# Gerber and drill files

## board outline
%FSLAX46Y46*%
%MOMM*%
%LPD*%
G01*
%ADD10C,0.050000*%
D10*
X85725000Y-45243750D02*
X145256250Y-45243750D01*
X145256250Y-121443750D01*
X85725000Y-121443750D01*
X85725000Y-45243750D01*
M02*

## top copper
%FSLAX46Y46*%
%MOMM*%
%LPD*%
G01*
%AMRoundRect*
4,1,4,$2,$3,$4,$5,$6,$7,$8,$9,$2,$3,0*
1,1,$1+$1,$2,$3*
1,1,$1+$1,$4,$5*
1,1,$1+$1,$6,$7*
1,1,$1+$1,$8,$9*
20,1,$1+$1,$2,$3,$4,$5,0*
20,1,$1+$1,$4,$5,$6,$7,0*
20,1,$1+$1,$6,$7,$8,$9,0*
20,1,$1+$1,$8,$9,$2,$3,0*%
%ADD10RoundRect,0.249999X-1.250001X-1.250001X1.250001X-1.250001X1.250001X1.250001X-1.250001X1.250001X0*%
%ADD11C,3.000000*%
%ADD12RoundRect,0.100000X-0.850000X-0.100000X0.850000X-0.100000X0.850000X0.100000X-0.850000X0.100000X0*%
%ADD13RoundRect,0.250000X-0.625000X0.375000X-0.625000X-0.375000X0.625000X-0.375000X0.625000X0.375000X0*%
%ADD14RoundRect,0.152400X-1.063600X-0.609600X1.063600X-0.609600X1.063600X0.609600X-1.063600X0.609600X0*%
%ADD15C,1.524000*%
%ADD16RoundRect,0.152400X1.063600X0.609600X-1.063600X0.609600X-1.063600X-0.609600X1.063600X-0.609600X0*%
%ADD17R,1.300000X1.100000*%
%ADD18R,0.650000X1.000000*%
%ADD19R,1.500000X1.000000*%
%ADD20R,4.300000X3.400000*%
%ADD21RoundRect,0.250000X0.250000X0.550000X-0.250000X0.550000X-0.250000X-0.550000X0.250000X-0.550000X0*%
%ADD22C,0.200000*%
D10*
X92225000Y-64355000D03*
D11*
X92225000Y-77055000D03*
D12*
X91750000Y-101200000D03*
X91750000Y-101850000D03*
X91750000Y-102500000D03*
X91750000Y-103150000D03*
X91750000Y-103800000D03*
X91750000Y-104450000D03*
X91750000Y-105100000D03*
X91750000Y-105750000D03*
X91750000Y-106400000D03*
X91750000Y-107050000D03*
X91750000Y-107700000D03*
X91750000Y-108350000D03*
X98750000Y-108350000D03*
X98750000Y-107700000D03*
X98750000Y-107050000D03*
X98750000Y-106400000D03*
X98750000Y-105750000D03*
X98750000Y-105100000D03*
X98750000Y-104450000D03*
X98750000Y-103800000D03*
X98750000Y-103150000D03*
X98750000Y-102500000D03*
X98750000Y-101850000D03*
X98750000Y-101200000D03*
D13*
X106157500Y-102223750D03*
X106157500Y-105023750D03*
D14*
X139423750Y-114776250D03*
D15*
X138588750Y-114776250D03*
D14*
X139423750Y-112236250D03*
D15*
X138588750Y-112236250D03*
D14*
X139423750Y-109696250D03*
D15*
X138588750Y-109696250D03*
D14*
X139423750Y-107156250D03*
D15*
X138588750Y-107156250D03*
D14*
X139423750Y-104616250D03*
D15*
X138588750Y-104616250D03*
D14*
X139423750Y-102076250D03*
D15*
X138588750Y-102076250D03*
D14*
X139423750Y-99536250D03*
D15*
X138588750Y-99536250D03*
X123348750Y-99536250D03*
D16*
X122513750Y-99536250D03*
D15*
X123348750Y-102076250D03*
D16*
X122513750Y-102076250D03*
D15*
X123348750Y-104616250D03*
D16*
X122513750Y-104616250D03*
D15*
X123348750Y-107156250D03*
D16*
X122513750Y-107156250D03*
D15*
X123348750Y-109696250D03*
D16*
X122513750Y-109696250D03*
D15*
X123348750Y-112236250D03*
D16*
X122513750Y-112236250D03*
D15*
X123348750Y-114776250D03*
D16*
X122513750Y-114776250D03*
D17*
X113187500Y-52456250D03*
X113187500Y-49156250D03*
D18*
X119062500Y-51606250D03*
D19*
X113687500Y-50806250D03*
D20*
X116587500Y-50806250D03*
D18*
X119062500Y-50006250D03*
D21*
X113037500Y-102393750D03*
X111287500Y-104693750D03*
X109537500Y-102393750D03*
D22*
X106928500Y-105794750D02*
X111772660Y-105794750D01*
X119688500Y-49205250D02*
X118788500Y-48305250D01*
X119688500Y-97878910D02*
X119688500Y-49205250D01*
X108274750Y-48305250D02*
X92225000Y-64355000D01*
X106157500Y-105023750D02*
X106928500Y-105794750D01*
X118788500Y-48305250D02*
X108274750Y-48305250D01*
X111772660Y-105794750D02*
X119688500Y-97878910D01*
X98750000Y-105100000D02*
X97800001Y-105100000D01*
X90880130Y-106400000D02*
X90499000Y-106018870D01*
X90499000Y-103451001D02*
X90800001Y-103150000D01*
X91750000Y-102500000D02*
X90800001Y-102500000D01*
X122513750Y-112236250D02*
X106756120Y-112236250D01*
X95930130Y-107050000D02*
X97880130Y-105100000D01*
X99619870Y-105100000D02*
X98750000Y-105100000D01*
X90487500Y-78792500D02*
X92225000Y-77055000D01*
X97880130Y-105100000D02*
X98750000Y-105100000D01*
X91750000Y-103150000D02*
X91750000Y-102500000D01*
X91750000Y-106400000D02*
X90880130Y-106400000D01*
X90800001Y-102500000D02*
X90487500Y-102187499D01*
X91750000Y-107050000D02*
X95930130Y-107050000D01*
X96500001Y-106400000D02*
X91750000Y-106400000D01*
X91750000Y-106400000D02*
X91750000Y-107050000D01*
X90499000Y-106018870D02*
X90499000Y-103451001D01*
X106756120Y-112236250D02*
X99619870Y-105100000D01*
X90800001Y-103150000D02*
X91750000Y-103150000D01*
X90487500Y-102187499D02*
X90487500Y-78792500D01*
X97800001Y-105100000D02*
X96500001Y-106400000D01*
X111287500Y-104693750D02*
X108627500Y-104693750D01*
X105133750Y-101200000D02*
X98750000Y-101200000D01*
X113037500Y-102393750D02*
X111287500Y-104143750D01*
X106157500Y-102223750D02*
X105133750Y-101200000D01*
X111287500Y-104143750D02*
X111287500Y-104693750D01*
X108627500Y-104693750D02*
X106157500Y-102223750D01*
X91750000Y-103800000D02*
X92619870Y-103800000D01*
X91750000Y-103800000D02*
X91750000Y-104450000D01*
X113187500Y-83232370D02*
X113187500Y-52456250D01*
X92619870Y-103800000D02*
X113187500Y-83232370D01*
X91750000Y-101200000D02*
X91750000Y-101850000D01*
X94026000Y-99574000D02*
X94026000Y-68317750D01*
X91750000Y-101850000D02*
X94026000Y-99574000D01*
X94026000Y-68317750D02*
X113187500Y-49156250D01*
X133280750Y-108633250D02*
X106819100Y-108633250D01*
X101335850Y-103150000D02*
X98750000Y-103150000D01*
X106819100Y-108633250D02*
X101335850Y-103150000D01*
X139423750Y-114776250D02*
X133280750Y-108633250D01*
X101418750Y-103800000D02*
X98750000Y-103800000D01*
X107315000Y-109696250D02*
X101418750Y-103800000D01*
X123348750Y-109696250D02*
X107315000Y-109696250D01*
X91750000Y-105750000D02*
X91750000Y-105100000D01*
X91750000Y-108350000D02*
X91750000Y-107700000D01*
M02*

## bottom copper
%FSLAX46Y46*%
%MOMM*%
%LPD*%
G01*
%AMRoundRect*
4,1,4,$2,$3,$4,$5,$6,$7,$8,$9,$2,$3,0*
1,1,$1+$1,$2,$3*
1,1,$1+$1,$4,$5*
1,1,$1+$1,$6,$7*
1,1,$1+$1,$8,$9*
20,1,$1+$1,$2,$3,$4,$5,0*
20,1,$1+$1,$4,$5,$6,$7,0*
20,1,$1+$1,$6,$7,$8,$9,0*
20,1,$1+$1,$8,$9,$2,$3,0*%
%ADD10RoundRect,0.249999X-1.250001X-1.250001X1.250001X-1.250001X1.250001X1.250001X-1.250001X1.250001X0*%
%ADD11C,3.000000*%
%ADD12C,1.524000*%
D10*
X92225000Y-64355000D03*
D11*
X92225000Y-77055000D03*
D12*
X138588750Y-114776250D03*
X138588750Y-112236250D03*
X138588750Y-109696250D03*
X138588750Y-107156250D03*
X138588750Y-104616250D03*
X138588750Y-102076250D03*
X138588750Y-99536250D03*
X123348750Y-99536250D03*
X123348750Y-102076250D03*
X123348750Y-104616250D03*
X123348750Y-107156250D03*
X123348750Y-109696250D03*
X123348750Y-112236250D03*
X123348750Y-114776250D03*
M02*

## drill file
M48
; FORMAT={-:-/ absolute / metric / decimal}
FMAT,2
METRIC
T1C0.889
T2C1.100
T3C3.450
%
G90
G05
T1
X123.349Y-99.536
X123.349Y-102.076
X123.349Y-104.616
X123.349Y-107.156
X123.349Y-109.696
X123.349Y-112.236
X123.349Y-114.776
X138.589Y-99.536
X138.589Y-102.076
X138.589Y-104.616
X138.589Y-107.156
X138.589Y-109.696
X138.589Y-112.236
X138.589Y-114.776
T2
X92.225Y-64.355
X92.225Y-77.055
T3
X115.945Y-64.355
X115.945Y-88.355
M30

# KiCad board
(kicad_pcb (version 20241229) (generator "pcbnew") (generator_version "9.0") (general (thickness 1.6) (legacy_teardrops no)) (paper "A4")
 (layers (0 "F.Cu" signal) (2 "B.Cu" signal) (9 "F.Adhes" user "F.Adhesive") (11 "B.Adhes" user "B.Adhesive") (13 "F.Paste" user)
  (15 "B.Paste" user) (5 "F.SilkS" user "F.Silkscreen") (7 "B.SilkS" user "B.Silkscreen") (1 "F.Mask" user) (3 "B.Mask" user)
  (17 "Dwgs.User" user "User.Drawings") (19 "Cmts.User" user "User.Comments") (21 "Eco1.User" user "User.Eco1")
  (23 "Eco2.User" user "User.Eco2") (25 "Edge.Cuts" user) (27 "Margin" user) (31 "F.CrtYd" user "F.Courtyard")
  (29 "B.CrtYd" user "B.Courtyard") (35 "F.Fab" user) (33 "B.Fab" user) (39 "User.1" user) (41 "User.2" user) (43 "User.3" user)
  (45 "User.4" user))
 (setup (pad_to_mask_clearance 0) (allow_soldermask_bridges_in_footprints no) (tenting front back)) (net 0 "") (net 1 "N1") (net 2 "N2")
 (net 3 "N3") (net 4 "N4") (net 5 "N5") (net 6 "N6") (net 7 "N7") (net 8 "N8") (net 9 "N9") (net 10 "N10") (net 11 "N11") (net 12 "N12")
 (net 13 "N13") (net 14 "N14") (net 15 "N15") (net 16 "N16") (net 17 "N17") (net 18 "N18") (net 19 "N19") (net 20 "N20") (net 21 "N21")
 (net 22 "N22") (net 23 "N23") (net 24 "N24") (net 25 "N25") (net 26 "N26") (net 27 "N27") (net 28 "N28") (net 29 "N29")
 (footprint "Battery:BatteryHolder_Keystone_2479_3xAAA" (layer "F.Cu") (at 92.225 64.355)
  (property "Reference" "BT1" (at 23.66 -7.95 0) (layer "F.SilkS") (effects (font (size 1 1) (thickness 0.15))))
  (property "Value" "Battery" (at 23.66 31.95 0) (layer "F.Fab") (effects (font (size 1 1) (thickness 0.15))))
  (pad "" np_thru_hole circle (at 23.72 0) (size 3.45 3.45) (drill 3.45) (layers "*.Cu" "*.Mask"))
  (pad "" np_thru_hole circle (at 23.72 24) (size 3.45 3.45) (drill 3.45) (layers "*.Cu" "*.Mask"))
  (pad "1" thru_hole roundrect (at 0 0) (size 3 3) (drill 1.1) (layers "*.Cu" "*.Mask") (remove_unused_layers no)
   (roundrect_rratio 0.083333) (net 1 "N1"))
  (pad "2" thru_hole circle (at 0 12.7) (size 3 3) (drill 1.1) (layers "*.Cu" "*.Mask") (remove_unused_layers no) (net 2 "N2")))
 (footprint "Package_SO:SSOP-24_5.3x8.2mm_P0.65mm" (layer "F.Cu") (at 95.25 104.775)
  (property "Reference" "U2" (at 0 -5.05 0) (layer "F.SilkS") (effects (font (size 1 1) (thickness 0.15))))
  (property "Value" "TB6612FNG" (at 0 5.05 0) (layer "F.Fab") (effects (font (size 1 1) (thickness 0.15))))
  (pad "1" smd roundrect (at -3.5 -3.575) (size 1.9 0.4) (layers "F.Cu" "F.Mask" "F.Paste") (roundrect_rratio 0.25) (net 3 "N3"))
  (pad "2" smd roundrect (at -3.5 -2.925) (size 1.9 0.4) (layers "F.Cu" "F.Mask" "F.Paste") (roundrect_rratio 0.25) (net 3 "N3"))
  (pad "3" smd roundrect (at -3.5 -2.275) (size 1.9 0.4) (layers "F.Cu" "F.Mask" "F.Paste") (roundrect_rratio 0.25) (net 2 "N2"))
  (pad "4" smd roundrect (at -3.5 -1.625) (size 1.9 0.4) (layers "F.Cu" "F.Mask" "F.Paste") (roundrect_rratio 0.25) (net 2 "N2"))
  (pad "5" smd roundrect (at -3.5 -0.975) (size 1.9 0.4) (layers "F.Cu" "F.Mask" "F.Paste") (roundrect_rratio 0.25) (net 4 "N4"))
  (pad "6" smd roundrect (at -3.5 -0.325) (size 1.9 0.4) (layers "F.Cu" "F.Mask" "F.Paste") (roundrect_rratio 0.25) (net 4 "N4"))
  (pad "7" smd roundrect (at -3.5 0.325) (size 1.9 0.4) (layers "F.Cu" "F.Mask" "F.Paste") (roundrect_rratio 0.25) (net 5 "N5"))
  (pad "8" smd roundrect (at -3.5 0.975) (size 1.9 0.4) (layers "F.Cu" "F.Mask" "F.Paste") (roundrect_rratio 0.25) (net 5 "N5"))
  (pad "9" smd roundrect (at -3.5 1.625) (size 1.9 0.4) (layers "F.Cu" "F.Mask" "F.Paste") (roundrect_rratio 0.25) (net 2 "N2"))
  (pad "10" smd roundrect (at -3.5 2.275) (size 1.9 0.4) (layers "F.Cu" "F.Mask" "F.Paste") (roundrect_rratio 0.25) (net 2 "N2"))
  (pad "11" smd roundrect (at -3.5 2.925) (size 1.9 0.4) (layers "F.Cu" "F.Mask" "F.Paste") (roundrect_rratio 0.25) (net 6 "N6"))
  (pad "12" smd roundrect (at -3.5 3.575) (size 1.9 0.4) (layers "F.Cu" "F.Mask" "F.Paste") (roundrect_rratio 0.25) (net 6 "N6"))
  (pad "13" smd roundrect (at 3.5 3.575) (size 1.9 0.4) (layers "F.Cu" "F.Mask" "F.Paste") (roundrect_rratio 0.25) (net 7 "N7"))
  (pad "14" smd roundrect (at 3.5 2.925) (size 1.9 0.4) (layers "F.Cu" "F.Mask" "F.Paste") (roundrect_rratio 0.25) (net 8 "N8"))
  (pad "15" smd roundrect (at 3.5 2.275) (size 1.9 0.4) (layers "F.Cu" "F.Mask" "F.Paste") (roundrect_rratio 0.25) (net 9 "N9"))
  (pad "16" smd roundrect (at 3.5 1.625) (size 1.9 0.4) (layers "F.Cu" "F.Mask" "F.Paste") (roundrect_rratio 0.25) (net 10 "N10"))
  (pad "17" smd roundrect (at 3.5 0.975) (size 1.9 0.4) (layers "F.Cu" "F.Mask" "F.Paste") (roundrect_rratio 0.25) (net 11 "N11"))
  (pad "18" smd roundrect (at 3.5 0.325) (size 1.9 0.4) (layers "F.Cu" "F.Mask" "F.Paste") (roundrect_rratio 0.25) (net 2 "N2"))
  (pad "19" smd roundrect (at 3.5 -0.325) (size 1.9 0.4) (layers "F.Cu" "F.Mask" "F.Paste") (roundrect_rratio 0.25) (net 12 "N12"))
  (pad "20" smd roundrect (at 3.5 -0.975) (size 1.9 0.4) (layers "F.Cu" "F.Mask" "F.Paste") (roundrect_rratio 0.25) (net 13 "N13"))
  (pad "21" smd roundrect (at 3.5 -1.625) (size 1.9 0.4) (layers "F.Cu" "F.Mask" "F.Paste") (roundrect_rratio 0.25) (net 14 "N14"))
  (pad "22" smd roundrect (at 3.5 -2.275) (size 1.9 0.4) (layers "F.Cu" "F.Mask" "F.Paste") (roundrect_rratio 0.25) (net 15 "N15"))
  (pad "23" smd roundrect (at 3.5 -2.925) (size 1.9 0.4) (layers "F.Cu" "F.Mask" "F.Paste") (roundrect_rratio 0.25) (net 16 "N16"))
  (pad "24" smd roundrect (at 3.5 -3.575) (size 1.9 0.4) (layers "F.Cu" "F.Mask" "F.Paste") (roundrect_rratio 0.25) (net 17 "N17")))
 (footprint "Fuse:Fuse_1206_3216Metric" (layer "F.Cu") (at 106.1575 103.62375 -90)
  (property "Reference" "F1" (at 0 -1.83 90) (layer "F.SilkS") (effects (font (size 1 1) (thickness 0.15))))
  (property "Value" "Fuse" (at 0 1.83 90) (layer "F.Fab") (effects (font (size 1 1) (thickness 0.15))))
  (pad "1" smd roundrect (at -1.4 0 270) (size 1.25 1.75) (layers "F.Cu" "F.Mask" "F.Paste") (roundrect_rratio 0.2) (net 17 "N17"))
  (pad "2" smd roundrect (at 1.4 0 270) (size 1.25 1.75) (layers "F.Cu" "F.Mask" "F.Paste") (roundrect_rratio 0.2) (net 1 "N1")))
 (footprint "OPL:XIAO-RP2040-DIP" (layer "F.Cu") (at 130.96875 107.15625 180)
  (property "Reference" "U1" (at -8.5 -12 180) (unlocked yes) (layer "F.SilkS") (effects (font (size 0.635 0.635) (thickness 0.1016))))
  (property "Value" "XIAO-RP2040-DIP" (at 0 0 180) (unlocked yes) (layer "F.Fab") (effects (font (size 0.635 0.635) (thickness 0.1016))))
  (pad "1" smd roundrect (at -8.455 -7.62) (size 2.432 1.524) (layers "F.Cu" "F.Mask") (roundrect_rratio 0.1) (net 14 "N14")
   (thermal_bridge_angle 45))
  (pad "1" thru_hole circle (at -7.62 -7.62) (size 1.524 1.524) (drill 0.889) (layers "*.Cu" "*.Mask") (remove_unused_layers no)
   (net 14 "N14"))
  (pad "2" smd roundrect (at -8.455 -5.08) (size 2.432 1.524) (layers "F.Cu" "F.Mask") (roundrect_rratio 0.1) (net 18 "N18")
   (thermal_bridge_angle 45))
  (pad "2" thru_hole circle (at -7.62 -5.08) (size 1.524 1.524) (drill 0.889) (layers "*.Cu" "*.Mask") (remove_unused_layers no)
   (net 18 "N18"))
  (pad "3" smd roundrect (at -8.455 -2.54) (size 2.432 1.524) (layers "F.Cu" "F.Mask") (roundrect_rratio 0.1) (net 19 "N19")
   (thermal_bridge_angle 45))
  (pad "3" thru_hole circle (at -7.62 -2.54) (size 1.524 1.524) (drill 0.889) (layers "*.Cu" "*.Mask") (remove_unused_layers no)
   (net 19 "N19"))
  (pad "4" smd roundrect (at -8.455 0) (size 2.432 1.524) (layers "F.Cu" "F.Mask") (roundrect_rratio 0.1) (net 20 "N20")
   (thermal_bridge_angle 45))
  (pad "4" thru_hole circle (at -7.62 0) (size 1.524 1.524) (drill 0.889) (layers "*.Cu" "*.Mask") (remove_unused_layers no) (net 20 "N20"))
  (pad "5" smd roundrect (at -8.455 2.54) (size 2.432 1.524) (layers "F.Cu" "F.Mask") (roundrect_rratio 0.1) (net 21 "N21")
   (thermal_bridge_angle 45))
  (pad "5" thru_hole circle (at -7.62 2.54) (size 1.524 1.524) (drill 0.889) (layers "*.Cu" "*.Mask") (remove_unused_layers no)
   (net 21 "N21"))
  (pad "6" smd roundrect (at -8.455 5.08) (size 2.432 1.524) (layers "F.Cu" "F.Mask") (roundrect_rratio 0.1) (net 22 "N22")
   (thermal_bridge_angle 45))
  (pad "6" thru_hole circle (at -7.62 5.08) (size 1.524 1.524) (drill 0.889) (layers "*.Cu" "*.Mask") (remove_unused_layers no)
   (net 22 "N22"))
  (pad "7" smd roundrect (at -8.455 7.62) (size 2.432 1.524) (layers "F.Cu" "F.Mask") (roundrect_rratio 0.1) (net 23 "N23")
   (thermal_bridge_angle 45))
  (pad "7" thru_hole circle (at -7.62 7.62) (size 1.524 1.524) (drill 0.889) (layers "*.Cu" "*.Mask") (remove_unused_layers no)
   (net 23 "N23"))
  (pad "8" thru_hole circle (at 7.62 7.62 180) (size 1.524 1.524) (drill 0.889) (layers "*.Cu" "*.Mask") (remove_unused_layers no)
   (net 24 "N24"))
  (pad "8" smd roundrect (at 8.455 7.62 180) (size 2.432 1.524) (layers "F.Cu" "F.Mask") (roundrect_rratio 0.1) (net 24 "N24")
   (thermal_bridge_angle 45))
  (pad "9" thru_hole circle (at 7.62 5.08 180) (size 1.524 1.524) (drill 0.889) (layers "*.Cu" "*.Mask") (remove_unused_layers no)
   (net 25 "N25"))
  (pad "9" smd roundrect (at 8.455 5.08 180) (size 2.432 1.524) (layers "F.Cu" "F.Mask") (roundrect_rratio 0.1) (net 25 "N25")
   (thermal_bridge_angle 45))
  (pad "10" thru_hole circle (at 7.62 2.54 180) (size 1.524 1.524) (drill 0.889) (layers "*.Cu" "*.Mask") (remove_unused_layers no)
   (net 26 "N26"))
  (pad "10" smd roundrect (at 8.455 2.54 180) (size 2.432 1.524) (layers "F.Cu" "F.Mask") (roundrect_rratio 0.1) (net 26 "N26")
   (thermal_bridge_angle 45))
  (pad "11" thru_hole circle (at 7.62 0 180) (size 1.524 1.524) (drill 0.889) (layers "*.Cu" "*.Mask") (remove_unused_layers no)
   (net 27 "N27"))
  (pad "11" smd roundrect (at 8.455 0 180) (size 2.432 1.524) (layers "F.Cu" "F.Mask") (roundrect_rratio 0.1) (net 27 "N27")
   (thermal_bridge_angle 45))
  (pad "12" thru_hole circle (at 7.62 -2.54 180) (size 1.524 1.524) (drill 0.889) (layers "*.Cu" "*.Mask") (remove_unused_layers no)
   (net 13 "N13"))
  (pad "12" smd roundrect (at 8.455 -2.54 180) (size 2.432 1.524) (layers "F.Cu" "F.Mask") (roundrect_rratio 0.1) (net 13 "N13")
   (thermal_bridge_angle 45))
  (pad "13" thru_hole circle (at 7.62 -5.08 180) (size 1.524 1.524) (drill 0.889) (layers "*.Cu" "*.Mask") (remove_unused_layers no)
   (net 2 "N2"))
  (pad "13" smd roundrect (at 8.455 -5.08 180) (size 2.432 1.524) (layers "F.Cu" "F.Mask") (roundrect_rratio 0.1) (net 2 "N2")
   (thermal_bridge_angle 45))
  (pad "14" thru_hole circle (at 7.62 -7.62 180) (size 1.524 1.524) (drill 0.889) (layers "*.Cu" "*.Mask") (remove_unused_layers no)
   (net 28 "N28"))
  (pad "14" smd roundrect (at 8.455 -7.62 180) (size 2.432 1.524) (layers "F.Cu" "F.Mask") (roundrect_rratio 0.1) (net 28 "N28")
   (thermal_bridge_angle 45)))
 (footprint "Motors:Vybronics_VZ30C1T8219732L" (layer "F.Cu") (at 117.5375 50.80625 90)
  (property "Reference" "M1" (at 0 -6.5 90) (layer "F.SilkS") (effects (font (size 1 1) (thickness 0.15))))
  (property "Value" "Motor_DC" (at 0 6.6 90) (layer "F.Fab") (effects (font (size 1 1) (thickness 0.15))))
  (pad "" smd rect (at -0.85 -2.315) (size 1.07 1.4) (layers "F.Paste"))
  (pad "" smd rect (at -0.85 -0.905) (size 1.07 1.4) (layers "F.Paste"))
  (pad "" smd rect (at -0.85 0.505) (size 1.07 1.4) (layers "F.Paste"))
  (pad "" smd rect (at 0.85 -2.315) (size 1.07 1.4) (layers "F.Paste"))
  (pad "" smd rect (at 0.85 -0.905) (size 1.07 1.4) (layers "F.Paste"))
  (pad "" smd rect (at 0.85 0.505) (size 1.07 1.4) (layers "F.Paste"))
  (pad "1" smd rect (at -1.65 -4.35) (size 1.3 1.1) (layers "F.Cu" "F.Mask" "F.Paste") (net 4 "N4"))
  (pad "2" smd rect (at 1.65 -4.35) (size 1.3 1.1) (layers "F.Cu" "F.Mask" "F.Paste") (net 3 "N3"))
  (pad "SH" smd rect (at -0.8 1.525 90) (size 1 0.65) (layers "F.Cu" "F.Mask" "F.Paste"))
  (pad "SH" smd rect (at 0 -3.85) (size 1.5 1) (layers "F.Cu" "F.Mask" "F.Paste"))
  (pad "SH" smd rect (at 0 -0.95) (size 4.3 3.4) (layers "F.Cu" "F.Mask"))
  (pad "SH" smd rect (at 0.8 1.525 90) (size 1 0.65) (layers "F.Cu" "F.Mask" "F.Paste")))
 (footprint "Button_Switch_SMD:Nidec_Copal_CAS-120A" (layer "F.Cu") (at 111.2875 103.54375 -90)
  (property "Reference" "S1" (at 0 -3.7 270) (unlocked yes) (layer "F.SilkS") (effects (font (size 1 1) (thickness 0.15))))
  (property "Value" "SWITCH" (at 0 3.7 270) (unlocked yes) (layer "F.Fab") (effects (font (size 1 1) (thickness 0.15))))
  (pad "1" smd roundrect (at -1.15 -1.75 180) (size 1 1.6) (layers "F.Cu" "F.Mask" "F.Paste") (roundrect_rratio 0.25) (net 17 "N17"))
  (pad "2" smd roundrect (at 1.15 0 180) (size 1 1.6) (layers "F.Cu" "F.Mask" "F.Paste") (roundrect_rratio 0.25) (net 17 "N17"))
  (pad "3" smd roundrect (at -1.15 1.75 180) (size 1 1.6) (layers "F.Cu" "F.Mask" "F.Paste") (roundrect_rratio 0.25) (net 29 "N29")))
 (gr_rect (start 85.725 45.24375) (end 145.25625 121.44375) (stroke (width 0.05) (type default)) (fill no) (layer "Edge.Cuts"))
 (segment (start 106.9285 105.79475) (end 111.77266 105.79475) (width 0.2) (layer "F.Cu") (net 1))
 (segment (start 119.6885 49.20525) (end 118.7885 48.30525) (width 0.2) (layer "F.Cu") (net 1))
 (segment (start 119.6885 97.87891) (end 119.6885 49.20525) (width 0.2) (layer "F.Cu") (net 1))
 (segment (start 108.27475 48.30525) (end 92.225 64.355) (width 0.2) (layer "F.Cu") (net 1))
 (segment (start 106.1575 105.02375) (end 106.9285 105.79475) (width 0.2) (layer "F.Cu") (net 1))
 (segment (start 118.7885 48.30525) (end 108.27475 48.30525) (width 0.2) (layer "F.Cu") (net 1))
 (segment (start 111.77266 105.79475) (end 119.6885 97.87891) (width 0.2) (layer "F.Cu") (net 1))
 (segment (start 98.75 105.1) (end 97.800001 105.1) (width 0.2) (layer "F.Cu") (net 2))
 (segment (start 90.88013 106.4) (end 90.499 106.01887) (width 0.2) (layer "F.Cu") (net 2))
 (segment (start 90.499 103.451001) (end 90.800001 103.15) (width 0.2) (layer "F.Cu") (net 2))
 (segment (start 91.75 102.5) (end 90.800001 102.5) (width 0.2) (layer "F.Cu") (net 2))
 (segment (start 122.51375 112.23625) (end 106.75612 112.23625) (width 0.2) (layer "F.Cu") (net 2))
 (segment (start 95.93013 107.05) (end 97.88013 105.1) (width 0.2) (layer "F.Cu") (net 2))
 (segment (start 99.61987 105.1) (end 98.75 105.1) (width 0.2) (layer "F.Cu") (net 2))
 (segment (start 90.4875 78.7925) (end 92.225 77.055) (width 0.2) (layer "F.Cu") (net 2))
 (segment (start 97.88013 105.1) (end 98.75 105.1) (width 0.2) (layer "F.Cu") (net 2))
 (segment (start 91.75 103.15) (end 91.75 102.5) (width 0.2) (layer "F.Cu") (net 2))
 (segment (start 91.75 106.4) (end 90.88013 106.4) (width 0.2) (layer "F.Cu") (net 2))
 (segment (start 90.800001 102.5) (end 90.4875 102.187499) (width 0.2) (layer "F.Cu") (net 2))
 (segment (start 91.75 107.05) (end 95.93013 107.05) (width 0.2) (layer "F.Cu") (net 2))
 (segment (start 96.500001 106.4) (end 91.75 106.4) (width 0.2) (layer "F.Cu") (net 2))
 (segment (start 91.75 106.4) (end 91.75 107.05) (width 0.2) (layer "F.Cu") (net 2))
 (segment (start 90.499 106.01887) (end 90.499 103.451001) (width 0.2) (layer "F.Cu") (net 2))
 (segment (start 106.75612 112.23625) (end 99.61987 105.1) (width 0.2) (layer "F.Cu") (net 2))
 (segment (start 90.800001 103.15) (end 91.75 103.15) (width 0.2) (layer "F.Cu") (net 2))
 (segment (start 90.4875 102.187499) (end 90.4875 78.7925) (width 0.2) (layer "F.Cu") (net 2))
 (segment (start 97.800001 105.1) (end 96.500001 106.4) (width 0.2) (layer "F.Cu") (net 2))
 (segment (start 111.2875 104.69375) (end 108.6275 104.69375) (width 0.2) (layer "F.Cu") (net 17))
 (segment (start 105.13375 101.2) (end 98.75 101.2) (width 0.2) (layer "F.Cu") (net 17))
 (segment (start 113.0375 102.39375) (end 111.2875 104.14375) (width 0.2) (layer "F.Cu") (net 17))
 (segment (start 106.1575 102.22375) (end 105.13375 101.2) (width 0.2) (layer "F.Cu") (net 17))
 (segment (start 111.2875 104.14375) (end 111.2875 104.69375) (width 0.2) (layer "F.Cu") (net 17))
 (segment (start 108.6275 104.69375) (end 106.1575 102.22375) (width 0.2) (layer "F.Cu") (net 17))
 (segment (start 91.75 103.8) (end 92.61987 103.8) (width 0.2) (layer "F.Cu") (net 4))
 (segment (start 91.75 103.8) (end 91.75 104.45) (width 0.2) (layer "F.Cu") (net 4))
 (segment (start 113.1875 83.23237) (end 113.1875 52.45625) (width 0.2) (layer "F.Cu") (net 4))
 (segment (start 92.61987 103.8) (end 113.1875 83.23237) (width 0.2) (layer "F.Cu") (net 4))
 (segment (start 91.75 101.2) (end 91.75 101.85) (width 0.2) (layer "F.Cu") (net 3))
 (segment (start 94.026 99.574) (end 94.026 68.31775) (width 0.2) (layer "F.Cu") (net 3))
 (segment (start 91.75 101.85) (end 94.026 99.574) (width 0.2) (layer "F.Cu") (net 3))
 (segment (start 94.026 68.31775) (end 113.1875 49.15625) (width 0.2) (layer "F.Cu") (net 3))
 (segment (start 133.28075 108.63325) (end 106.8191 108.63325) (width 0.2) (layer "F.Cu") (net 14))
 (segment (start 101.33585 103.15) (end 98.75 103.15) (width 0.2) (layer "F.Cu") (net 14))
 (segment (start 106.8191 108.63325) (end 101.33585 103.15) (width 0.2) (layer "F.Cu") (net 14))
 (segment (start 139.42375 114.77625) (end 133.28075 108.63325) (width 0.2) (layer "F.Cu") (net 14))
 (segment (start 101.41875 103.8) (end 98.75 103.8) (width 0.2) (layer "F.Cu") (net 13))
 (segment (start 107.315 109.69625) (end 101.41875 103.8) (width 0.2) (layer "F.Cu") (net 13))
 (segment (start 123.34875 109.69625) (end 107.315 109.69625) (width 0.2) (layer "F.Cu") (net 13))
 (segment (start 91.75 105.75) (end 91.75 105.1) (width 0.2) (layer "F.Cu") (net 5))
 (segment (start 91.75 108.35) (end 91.75 107.7) (width 0.2) (layer "F.Cu") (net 6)))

